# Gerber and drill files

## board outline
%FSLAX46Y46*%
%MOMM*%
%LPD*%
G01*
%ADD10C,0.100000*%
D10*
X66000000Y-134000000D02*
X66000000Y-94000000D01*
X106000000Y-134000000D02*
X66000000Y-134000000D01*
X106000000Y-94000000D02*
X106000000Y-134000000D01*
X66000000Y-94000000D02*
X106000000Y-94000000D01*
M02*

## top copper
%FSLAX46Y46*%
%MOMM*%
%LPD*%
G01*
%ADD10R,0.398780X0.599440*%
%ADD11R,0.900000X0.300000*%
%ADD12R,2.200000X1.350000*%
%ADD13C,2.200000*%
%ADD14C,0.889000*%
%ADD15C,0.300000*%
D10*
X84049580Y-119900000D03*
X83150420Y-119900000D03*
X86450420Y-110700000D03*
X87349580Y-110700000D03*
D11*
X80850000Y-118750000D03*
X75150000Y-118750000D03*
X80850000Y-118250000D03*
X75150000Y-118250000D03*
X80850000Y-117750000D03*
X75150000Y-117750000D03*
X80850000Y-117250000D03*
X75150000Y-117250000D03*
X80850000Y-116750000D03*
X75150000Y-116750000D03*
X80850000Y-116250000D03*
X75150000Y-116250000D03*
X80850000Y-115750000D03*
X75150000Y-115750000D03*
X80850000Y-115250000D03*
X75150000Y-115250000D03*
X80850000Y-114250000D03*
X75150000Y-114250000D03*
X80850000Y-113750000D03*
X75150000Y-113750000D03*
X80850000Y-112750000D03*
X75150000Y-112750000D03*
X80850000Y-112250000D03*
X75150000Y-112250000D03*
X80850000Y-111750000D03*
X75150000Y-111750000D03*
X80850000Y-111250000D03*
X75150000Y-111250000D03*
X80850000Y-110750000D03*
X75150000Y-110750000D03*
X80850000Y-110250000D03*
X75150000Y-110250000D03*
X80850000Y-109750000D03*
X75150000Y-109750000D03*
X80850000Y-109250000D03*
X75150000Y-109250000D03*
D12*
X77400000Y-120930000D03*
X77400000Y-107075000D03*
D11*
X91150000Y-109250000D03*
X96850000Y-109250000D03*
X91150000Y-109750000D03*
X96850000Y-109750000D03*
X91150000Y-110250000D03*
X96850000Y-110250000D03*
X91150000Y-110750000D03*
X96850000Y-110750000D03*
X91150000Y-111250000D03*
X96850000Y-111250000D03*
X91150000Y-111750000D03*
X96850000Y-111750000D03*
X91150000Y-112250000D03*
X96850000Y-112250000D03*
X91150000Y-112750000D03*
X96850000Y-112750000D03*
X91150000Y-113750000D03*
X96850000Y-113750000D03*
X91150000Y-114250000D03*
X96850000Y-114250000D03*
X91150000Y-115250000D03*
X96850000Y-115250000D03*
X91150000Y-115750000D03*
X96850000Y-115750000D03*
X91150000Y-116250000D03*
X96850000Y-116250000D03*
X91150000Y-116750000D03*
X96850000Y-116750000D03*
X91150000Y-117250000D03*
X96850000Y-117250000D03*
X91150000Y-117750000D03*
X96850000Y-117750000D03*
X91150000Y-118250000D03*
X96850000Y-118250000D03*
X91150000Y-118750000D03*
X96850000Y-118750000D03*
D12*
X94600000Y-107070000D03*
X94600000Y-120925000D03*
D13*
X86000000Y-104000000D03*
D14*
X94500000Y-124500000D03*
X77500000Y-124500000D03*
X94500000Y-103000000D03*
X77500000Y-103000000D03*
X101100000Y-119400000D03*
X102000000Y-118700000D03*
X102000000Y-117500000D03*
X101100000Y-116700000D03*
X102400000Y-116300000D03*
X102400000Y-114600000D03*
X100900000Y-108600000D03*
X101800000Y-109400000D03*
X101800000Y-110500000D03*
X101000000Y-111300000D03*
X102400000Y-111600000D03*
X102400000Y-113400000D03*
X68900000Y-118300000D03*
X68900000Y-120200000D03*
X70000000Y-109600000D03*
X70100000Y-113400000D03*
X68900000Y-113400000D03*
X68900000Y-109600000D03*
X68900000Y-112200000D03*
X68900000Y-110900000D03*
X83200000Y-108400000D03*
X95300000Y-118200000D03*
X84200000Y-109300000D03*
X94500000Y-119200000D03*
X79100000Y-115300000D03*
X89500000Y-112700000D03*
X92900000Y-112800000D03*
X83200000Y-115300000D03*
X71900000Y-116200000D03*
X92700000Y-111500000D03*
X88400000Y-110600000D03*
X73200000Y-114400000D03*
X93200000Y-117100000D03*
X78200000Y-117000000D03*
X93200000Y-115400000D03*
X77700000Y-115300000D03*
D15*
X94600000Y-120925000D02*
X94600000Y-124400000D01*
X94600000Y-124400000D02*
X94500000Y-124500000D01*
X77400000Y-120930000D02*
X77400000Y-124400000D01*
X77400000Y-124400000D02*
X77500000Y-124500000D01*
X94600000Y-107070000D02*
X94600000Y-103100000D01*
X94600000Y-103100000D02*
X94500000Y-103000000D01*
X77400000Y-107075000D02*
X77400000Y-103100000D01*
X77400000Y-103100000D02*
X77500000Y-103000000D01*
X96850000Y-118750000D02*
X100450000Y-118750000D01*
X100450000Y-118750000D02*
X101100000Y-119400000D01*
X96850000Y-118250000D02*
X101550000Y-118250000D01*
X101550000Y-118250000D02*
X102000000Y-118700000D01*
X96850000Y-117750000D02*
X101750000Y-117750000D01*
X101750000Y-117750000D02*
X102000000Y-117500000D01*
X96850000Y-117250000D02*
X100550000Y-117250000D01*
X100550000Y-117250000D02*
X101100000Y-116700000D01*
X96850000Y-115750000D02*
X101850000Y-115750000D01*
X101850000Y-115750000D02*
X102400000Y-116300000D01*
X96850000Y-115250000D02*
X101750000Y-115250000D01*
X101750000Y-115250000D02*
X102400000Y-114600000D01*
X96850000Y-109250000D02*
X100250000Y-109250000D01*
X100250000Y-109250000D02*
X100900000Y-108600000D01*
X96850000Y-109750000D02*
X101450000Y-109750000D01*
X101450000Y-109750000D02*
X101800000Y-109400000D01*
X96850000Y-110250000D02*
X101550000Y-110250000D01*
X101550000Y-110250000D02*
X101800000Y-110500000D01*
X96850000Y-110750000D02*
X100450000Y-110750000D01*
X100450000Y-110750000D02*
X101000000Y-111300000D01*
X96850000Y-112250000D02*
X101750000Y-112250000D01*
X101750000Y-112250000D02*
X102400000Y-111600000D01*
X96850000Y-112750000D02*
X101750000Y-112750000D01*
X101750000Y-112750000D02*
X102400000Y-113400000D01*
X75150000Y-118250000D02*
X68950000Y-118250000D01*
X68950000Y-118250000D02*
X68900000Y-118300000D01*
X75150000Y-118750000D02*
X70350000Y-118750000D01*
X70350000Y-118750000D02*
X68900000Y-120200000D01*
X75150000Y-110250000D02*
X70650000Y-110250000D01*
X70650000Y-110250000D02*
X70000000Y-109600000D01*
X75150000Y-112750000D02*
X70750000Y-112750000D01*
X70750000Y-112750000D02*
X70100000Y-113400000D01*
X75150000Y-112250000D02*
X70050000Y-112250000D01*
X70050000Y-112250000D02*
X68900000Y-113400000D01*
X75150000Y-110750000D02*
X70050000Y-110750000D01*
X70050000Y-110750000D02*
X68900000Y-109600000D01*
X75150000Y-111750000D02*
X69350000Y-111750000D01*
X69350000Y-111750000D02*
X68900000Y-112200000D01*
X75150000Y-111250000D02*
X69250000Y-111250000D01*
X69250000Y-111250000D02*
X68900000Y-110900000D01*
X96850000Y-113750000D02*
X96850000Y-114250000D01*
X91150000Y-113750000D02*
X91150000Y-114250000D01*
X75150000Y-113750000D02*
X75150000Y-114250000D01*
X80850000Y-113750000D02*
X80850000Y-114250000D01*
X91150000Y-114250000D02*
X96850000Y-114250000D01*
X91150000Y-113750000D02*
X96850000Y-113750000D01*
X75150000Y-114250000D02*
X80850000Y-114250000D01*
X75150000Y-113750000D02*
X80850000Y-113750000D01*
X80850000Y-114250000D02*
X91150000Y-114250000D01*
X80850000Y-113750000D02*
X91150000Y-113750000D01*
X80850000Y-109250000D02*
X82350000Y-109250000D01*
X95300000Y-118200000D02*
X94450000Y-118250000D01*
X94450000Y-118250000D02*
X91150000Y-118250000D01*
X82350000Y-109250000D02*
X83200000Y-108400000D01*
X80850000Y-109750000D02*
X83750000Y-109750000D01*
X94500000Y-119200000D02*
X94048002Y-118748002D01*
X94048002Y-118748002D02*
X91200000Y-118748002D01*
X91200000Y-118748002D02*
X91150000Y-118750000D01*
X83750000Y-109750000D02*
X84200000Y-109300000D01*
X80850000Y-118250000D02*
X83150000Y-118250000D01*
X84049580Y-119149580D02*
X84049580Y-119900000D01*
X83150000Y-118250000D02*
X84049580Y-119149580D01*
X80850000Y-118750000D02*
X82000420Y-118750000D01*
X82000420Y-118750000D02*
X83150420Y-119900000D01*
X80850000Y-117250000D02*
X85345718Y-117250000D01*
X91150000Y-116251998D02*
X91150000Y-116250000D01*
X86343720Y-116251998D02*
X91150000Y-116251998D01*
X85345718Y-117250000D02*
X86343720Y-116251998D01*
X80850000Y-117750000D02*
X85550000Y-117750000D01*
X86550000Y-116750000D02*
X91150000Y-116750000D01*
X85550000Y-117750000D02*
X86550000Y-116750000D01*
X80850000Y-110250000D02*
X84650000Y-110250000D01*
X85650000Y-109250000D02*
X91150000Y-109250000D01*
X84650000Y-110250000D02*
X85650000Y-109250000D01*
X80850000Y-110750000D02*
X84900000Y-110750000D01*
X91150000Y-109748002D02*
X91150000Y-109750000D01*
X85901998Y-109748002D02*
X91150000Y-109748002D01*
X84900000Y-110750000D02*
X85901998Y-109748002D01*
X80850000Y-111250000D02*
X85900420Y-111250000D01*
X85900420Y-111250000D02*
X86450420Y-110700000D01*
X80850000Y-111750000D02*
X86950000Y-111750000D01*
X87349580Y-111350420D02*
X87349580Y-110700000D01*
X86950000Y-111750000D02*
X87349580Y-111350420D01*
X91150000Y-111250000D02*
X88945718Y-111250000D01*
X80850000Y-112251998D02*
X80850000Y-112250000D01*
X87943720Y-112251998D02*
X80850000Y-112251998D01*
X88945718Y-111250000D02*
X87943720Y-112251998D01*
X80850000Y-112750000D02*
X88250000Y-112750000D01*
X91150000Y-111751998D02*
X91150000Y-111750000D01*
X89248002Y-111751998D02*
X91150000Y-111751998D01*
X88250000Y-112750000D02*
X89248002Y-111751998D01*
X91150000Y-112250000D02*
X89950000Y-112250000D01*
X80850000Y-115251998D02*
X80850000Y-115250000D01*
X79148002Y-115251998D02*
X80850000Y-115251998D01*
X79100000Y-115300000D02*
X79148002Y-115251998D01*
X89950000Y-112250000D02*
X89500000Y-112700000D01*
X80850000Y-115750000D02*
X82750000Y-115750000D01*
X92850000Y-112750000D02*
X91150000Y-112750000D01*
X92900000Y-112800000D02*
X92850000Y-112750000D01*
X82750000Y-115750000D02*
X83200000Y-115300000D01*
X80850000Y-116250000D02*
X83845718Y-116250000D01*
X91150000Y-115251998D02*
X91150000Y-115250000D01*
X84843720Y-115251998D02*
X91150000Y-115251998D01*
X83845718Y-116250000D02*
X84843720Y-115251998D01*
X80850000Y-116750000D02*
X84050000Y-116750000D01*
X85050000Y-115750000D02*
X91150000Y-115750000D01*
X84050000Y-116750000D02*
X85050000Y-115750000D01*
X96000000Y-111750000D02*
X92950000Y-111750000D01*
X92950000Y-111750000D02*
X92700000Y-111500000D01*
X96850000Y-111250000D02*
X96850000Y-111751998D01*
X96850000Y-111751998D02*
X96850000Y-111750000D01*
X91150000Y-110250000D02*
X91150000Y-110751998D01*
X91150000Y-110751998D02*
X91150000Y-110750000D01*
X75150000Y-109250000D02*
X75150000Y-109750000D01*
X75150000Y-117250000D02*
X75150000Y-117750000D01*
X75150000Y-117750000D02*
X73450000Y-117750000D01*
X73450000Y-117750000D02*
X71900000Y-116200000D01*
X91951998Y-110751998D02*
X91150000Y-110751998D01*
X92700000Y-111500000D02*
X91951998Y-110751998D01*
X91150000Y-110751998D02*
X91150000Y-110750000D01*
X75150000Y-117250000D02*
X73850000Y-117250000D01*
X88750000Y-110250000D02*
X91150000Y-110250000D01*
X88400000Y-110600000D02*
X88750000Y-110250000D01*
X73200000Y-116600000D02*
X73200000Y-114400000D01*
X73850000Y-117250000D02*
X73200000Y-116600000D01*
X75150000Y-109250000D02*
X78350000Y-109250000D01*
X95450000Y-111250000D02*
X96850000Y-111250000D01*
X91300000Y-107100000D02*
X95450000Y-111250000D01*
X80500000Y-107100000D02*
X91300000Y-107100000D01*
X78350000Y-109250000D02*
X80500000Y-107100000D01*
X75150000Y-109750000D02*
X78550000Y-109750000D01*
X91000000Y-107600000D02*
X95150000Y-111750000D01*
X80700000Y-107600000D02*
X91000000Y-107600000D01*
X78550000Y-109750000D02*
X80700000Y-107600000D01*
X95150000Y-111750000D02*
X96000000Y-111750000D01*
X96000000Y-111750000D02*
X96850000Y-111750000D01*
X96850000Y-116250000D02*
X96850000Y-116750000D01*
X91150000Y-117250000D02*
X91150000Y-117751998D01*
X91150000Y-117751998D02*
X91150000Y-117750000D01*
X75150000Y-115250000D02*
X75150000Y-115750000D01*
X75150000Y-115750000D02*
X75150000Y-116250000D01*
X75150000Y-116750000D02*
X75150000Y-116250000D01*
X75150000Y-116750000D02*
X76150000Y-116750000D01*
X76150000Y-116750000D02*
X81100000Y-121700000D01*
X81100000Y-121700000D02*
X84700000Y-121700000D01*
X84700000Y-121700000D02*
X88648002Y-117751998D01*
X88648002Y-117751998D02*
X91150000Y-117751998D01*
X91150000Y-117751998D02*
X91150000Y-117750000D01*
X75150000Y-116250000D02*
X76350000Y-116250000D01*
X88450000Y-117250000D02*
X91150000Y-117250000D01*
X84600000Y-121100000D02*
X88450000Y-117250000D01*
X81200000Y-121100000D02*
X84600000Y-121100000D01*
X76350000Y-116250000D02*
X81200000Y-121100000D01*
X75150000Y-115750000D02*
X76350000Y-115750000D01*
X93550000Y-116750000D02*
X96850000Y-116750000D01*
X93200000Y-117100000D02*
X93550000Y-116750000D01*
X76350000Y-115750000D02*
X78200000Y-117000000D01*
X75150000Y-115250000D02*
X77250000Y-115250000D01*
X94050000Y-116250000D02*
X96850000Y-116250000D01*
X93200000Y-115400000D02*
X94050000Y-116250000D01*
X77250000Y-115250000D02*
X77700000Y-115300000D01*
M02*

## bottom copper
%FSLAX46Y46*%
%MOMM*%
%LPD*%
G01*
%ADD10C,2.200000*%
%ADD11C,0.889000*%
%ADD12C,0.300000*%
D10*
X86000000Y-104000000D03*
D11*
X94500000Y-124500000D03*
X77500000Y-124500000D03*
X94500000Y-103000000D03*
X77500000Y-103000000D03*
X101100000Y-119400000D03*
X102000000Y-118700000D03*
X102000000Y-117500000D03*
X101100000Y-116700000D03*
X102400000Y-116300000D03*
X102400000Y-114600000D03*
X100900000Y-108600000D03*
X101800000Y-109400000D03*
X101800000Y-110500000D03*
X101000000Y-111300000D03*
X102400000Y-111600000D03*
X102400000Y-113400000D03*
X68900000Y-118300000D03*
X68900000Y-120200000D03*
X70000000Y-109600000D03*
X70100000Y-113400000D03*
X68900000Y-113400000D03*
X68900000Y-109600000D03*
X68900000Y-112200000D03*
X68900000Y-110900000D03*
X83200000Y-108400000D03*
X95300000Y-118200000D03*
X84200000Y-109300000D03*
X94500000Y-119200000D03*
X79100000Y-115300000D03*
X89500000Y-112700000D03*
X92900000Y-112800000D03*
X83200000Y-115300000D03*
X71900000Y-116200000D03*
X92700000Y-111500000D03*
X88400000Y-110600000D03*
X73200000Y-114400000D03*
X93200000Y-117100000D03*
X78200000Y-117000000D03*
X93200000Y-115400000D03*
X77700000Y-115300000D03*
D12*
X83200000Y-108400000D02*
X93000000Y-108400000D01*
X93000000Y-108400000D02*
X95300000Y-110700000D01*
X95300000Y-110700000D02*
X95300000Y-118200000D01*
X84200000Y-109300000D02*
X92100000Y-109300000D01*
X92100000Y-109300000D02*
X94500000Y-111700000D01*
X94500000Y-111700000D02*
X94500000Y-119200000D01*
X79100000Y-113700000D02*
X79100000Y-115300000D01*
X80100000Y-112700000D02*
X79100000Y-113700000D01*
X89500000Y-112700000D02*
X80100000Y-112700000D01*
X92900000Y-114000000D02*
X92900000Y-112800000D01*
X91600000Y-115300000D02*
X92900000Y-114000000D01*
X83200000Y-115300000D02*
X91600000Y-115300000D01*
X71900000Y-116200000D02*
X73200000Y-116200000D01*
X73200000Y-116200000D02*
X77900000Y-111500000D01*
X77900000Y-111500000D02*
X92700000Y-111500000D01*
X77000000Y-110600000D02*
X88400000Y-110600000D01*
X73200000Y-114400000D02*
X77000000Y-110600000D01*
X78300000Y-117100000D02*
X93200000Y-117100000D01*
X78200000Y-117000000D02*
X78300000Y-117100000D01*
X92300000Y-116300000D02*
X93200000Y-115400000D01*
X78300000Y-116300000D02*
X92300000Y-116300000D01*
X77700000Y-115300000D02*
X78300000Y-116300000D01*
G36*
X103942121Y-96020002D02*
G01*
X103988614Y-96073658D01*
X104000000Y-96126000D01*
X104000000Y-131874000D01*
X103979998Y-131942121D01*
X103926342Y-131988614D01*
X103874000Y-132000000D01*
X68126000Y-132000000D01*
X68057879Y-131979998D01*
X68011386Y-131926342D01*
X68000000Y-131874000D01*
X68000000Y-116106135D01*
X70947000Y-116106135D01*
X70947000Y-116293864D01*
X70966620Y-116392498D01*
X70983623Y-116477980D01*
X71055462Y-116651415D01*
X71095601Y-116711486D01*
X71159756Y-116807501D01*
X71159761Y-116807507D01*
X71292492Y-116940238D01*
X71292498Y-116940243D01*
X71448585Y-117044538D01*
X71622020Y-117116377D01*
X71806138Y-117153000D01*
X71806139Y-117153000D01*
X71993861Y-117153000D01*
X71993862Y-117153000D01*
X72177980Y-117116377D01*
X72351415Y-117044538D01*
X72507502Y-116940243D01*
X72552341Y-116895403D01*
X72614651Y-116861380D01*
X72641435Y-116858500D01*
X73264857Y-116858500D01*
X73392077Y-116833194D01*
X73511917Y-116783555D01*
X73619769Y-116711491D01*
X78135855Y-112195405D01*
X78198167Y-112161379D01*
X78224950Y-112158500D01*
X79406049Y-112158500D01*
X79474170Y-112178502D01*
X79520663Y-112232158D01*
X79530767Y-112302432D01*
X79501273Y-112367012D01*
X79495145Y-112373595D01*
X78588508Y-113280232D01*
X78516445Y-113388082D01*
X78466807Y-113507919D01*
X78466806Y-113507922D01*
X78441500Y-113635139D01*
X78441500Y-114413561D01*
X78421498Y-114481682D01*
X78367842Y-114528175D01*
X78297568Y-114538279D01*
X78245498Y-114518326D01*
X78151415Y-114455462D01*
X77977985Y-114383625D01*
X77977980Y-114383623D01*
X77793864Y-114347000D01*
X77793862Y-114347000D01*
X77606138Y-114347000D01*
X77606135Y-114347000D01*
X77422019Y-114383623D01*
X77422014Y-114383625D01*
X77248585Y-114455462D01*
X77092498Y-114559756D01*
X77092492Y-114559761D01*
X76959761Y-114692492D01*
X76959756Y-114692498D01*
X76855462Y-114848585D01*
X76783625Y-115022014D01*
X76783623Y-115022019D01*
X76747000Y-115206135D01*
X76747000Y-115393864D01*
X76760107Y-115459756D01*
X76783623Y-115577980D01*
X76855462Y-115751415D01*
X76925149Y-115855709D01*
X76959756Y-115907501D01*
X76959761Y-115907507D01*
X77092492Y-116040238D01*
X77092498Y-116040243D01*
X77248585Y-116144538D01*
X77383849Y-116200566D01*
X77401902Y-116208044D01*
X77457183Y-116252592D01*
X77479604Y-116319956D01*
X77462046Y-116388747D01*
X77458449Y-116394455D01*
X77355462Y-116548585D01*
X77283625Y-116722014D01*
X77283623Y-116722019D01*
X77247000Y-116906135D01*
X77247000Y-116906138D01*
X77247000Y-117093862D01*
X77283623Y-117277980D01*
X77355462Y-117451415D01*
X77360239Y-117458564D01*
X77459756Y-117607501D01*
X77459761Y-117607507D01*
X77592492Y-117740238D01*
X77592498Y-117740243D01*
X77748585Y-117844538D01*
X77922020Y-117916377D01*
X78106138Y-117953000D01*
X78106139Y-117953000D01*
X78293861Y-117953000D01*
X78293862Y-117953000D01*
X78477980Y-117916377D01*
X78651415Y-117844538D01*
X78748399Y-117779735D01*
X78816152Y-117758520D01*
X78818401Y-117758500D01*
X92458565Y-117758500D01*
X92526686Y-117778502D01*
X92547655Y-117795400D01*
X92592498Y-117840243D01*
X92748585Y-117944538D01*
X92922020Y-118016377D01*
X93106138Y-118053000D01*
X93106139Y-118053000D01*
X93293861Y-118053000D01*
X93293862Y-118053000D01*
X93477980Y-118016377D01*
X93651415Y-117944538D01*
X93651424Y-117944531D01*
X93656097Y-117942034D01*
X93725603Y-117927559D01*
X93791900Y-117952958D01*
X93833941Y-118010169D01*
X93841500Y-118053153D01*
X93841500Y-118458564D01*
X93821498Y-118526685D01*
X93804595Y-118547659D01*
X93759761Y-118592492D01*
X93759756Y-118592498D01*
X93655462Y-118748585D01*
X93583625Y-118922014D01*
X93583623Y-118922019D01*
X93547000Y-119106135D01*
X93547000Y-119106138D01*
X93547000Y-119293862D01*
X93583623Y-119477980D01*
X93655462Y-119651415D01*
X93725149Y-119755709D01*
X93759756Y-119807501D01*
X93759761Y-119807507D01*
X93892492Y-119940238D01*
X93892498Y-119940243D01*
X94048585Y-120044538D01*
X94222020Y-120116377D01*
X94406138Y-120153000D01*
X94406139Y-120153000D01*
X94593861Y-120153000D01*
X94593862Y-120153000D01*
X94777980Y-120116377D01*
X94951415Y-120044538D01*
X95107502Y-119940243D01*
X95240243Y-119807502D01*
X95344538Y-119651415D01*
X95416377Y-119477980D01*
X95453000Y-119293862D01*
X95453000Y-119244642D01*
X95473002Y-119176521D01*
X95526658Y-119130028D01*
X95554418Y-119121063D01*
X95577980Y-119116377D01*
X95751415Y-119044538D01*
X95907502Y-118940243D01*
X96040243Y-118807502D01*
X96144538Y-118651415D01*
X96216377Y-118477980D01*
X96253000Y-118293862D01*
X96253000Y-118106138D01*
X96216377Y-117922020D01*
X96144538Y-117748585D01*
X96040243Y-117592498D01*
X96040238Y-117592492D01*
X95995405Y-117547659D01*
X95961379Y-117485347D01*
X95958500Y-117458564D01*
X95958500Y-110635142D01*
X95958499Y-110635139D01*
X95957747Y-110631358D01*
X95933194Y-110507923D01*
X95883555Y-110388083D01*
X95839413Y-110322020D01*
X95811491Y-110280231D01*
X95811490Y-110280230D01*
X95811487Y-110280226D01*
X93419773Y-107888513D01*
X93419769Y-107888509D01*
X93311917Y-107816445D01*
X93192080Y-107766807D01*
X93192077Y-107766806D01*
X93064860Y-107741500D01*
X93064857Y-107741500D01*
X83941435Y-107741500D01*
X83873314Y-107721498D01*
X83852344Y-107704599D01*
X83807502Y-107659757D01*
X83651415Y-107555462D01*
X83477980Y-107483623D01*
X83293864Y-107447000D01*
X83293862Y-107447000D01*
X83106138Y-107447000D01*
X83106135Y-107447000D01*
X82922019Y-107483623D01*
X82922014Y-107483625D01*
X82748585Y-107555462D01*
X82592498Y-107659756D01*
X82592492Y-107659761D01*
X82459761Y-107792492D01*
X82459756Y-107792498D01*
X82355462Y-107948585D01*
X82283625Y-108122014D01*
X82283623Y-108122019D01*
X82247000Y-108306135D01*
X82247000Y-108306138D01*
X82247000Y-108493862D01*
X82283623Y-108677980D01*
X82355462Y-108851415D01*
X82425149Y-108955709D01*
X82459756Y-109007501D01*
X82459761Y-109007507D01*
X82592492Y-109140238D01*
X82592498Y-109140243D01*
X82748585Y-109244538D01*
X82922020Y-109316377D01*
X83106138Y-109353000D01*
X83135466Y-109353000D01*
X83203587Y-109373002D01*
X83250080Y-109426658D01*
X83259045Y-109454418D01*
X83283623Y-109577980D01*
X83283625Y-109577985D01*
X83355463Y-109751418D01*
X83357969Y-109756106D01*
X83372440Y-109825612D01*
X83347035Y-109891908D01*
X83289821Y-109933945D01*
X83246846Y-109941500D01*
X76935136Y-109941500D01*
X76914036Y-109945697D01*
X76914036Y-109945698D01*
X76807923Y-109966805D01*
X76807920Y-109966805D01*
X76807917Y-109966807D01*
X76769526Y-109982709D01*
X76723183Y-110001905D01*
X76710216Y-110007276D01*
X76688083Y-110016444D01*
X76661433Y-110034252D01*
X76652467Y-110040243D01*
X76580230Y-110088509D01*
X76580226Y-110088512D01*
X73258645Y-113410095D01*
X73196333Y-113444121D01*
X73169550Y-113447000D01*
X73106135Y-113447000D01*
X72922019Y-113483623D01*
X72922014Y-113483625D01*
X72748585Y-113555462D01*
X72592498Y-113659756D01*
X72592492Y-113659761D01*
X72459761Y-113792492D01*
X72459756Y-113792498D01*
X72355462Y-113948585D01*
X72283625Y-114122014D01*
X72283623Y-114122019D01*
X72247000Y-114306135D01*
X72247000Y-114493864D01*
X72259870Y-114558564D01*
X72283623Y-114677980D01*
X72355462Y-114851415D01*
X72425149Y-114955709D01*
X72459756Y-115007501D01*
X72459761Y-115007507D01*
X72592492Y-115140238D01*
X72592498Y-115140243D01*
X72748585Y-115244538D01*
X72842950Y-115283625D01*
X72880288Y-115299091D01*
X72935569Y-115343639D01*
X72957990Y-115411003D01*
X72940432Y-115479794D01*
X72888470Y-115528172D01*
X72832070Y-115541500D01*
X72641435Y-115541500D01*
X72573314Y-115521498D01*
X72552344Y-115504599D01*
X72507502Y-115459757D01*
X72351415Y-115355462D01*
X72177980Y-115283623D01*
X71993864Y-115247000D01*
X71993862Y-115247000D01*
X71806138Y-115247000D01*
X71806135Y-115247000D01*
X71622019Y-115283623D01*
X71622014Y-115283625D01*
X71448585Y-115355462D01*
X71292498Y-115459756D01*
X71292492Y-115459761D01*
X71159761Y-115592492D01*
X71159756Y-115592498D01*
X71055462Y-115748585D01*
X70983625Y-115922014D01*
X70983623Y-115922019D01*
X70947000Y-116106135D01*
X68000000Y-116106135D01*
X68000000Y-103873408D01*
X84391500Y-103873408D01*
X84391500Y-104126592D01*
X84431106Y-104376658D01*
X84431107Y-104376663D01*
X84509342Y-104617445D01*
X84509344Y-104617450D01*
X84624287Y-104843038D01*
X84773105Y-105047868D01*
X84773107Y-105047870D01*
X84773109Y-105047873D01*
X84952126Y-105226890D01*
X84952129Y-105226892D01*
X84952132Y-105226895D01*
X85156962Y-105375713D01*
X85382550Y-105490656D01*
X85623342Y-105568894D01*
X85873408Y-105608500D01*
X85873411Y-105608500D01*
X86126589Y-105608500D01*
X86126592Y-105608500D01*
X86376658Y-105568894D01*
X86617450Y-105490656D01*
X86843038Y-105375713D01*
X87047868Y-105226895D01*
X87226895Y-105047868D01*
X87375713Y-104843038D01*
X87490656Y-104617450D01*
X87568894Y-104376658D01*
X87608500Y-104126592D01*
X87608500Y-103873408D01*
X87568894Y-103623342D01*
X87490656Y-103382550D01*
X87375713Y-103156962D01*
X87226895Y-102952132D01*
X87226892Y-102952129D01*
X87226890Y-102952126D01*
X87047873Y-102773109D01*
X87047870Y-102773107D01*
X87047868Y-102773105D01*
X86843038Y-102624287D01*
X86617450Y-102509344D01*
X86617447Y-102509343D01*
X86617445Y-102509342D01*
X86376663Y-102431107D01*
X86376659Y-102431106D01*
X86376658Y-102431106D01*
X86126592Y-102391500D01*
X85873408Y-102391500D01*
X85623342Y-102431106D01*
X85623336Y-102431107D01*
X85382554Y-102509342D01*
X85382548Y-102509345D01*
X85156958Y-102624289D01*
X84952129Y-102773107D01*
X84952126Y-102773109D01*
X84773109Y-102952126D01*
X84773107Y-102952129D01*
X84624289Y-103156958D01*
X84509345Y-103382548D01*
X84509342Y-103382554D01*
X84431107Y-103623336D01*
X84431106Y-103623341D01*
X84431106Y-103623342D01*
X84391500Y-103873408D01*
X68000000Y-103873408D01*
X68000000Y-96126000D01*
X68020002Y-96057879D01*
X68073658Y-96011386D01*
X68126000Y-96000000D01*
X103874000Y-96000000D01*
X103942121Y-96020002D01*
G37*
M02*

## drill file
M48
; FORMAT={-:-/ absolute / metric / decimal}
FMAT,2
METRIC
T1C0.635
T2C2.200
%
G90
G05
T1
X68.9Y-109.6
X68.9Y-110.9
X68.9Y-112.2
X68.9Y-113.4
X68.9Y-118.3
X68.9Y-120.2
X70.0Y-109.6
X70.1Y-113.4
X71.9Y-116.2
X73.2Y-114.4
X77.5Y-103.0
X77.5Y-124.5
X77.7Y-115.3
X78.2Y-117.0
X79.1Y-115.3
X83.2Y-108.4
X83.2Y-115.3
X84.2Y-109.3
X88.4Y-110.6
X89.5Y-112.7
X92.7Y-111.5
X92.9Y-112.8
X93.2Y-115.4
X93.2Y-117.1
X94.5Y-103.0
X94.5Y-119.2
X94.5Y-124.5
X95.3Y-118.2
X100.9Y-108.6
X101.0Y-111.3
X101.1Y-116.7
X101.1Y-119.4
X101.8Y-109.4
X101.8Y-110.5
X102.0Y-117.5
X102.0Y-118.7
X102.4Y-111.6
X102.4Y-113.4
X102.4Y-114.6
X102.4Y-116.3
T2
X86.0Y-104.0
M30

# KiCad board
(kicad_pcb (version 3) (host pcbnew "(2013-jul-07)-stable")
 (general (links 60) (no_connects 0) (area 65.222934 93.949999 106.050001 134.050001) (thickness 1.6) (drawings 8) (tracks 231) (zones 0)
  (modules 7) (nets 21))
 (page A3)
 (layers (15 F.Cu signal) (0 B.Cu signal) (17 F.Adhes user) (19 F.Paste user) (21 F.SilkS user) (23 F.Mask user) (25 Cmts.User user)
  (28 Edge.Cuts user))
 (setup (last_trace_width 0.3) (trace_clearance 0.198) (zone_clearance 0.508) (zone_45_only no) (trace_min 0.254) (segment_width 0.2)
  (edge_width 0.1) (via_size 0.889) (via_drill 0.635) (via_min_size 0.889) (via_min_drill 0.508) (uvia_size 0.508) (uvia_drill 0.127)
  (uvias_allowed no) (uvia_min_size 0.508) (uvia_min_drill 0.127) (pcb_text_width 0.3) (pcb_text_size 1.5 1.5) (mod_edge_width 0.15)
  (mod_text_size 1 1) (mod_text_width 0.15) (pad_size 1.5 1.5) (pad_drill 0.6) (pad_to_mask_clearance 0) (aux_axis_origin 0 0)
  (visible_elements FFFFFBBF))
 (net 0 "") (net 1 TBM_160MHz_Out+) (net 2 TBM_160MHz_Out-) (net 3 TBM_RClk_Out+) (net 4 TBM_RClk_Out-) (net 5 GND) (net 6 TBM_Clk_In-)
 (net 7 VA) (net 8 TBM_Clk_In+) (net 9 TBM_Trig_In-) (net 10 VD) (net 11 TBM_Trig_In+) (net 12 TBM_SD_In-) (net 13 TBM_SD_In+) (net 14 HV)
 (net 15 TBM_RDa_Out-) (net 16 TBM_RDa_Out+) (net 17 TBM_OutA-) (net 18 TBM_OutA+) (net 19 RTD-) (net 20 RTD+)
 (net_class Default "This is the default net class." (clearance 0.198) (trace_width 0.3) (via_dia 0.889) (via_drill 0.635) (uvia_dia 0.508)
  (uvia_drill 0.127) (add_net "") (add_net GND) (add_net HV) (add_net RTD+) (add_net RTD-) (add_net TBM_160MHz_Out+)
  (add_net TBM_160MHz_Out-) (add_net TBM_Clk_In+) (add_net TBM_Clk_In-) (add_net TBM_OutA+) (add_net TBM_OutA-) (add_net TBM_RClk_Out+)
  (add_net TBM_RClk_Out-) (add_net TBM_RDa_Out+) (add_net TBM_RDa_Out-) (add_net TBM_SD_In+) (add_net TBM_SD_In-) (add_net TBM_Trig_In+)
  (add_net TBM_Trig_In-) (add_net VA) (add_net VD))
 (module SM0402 (layer F.Cu) (at 83.6 119.9 180)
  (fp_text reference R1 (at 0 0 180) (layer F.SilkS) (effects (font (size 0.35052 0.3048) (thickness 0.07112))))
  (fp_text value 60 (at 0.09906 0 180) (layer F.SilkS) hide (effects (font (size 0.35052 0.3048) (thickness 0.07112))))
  (pad 1 smd rect (at -0.44958 0 180) (size 0.39878 0.59944) (layers F.Cu F.Paste F.Mask) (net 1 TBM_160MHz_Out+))
  (pad 2 smd rect (at 0.44958 0 180) (size 0.39878 0.59944) (layers F.Cu F.Paste F.Mask) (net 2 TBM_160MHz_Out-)))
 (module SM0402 (layer F.Cu) (at 86.9 110.7)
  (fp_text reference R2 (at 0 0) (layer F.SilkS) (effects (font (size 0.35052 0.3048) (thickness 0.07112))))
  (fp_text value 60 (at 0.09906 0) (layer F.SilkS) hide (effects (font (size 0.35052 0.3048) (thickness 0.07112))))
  (pad 1 smd rect (at -0.44958 0) (size 0.39878 0.59944) (layers F.Cu F.Paste F.Mask) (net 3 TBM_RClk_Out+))
  (pad 2 smd rect (at 0.44958 0) (size 0.39878 0.59944) (layers F.Cu F.Paste F.Mask) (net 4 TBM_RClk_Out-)))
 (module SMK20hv (layer F.Cu) (at 78 114 90)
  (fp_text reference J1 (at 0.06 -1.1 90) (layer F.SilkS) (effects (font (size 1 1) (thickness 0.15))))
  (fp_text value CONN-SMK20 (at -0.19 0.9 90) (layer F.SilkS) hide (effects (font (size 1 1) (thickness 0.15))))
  (pad 1 smd rect (at -4.75 2.85 90) (size 0.3 0.9) (layers F.Cu F.Paste F.Mask) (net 2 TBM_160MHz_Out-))
  (pad 2 smd rect (at -4.75 -2.85 90) (size 0.3 0.9) (layers F.Cu F.Paste F.Mask) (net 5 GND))
  (pad 3 smd rect (at -4.25 2.85 90) (size 0.3 0.9) (layers F.Cu F.Paste F.Mask) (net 1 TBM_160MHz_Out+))
  (pad 4 smd rect (at -4.25 -2.85 90) (size 0.3 0.9) (layers F.Cu F.Paste F.Mask) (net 5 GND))
  (pad 5 smd rect (at -3.75 2.85 90) (size 0.3 0.9) (layers F.Cu F.Paste F.Mask) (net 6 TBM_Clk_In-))
  (pad 6 smd rect (at -3.75 -2.85 90) (size 0.3 0.9) (layers F.Cu F.Paste F.Mask) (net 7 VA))
  (pad 7 smd rect (at -3.25 2.85 90) (size 0.3 0.9) (layers F.Cu F.Paste F.Mask) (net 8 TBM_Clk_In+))
  (pad 8 smd rect (at -3.25 -2.85 90) (size 0.3 0.9) (layers F.Cu F.Paste F.Mask) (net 7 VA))
  (pad 9 smd rect (at -2.75 2.85 90) (size 0.3 0.9) (layers F.Cu F.Paste F.Mask) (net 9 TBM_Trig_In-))
  (pad 10 smd rect (at -2.75 -2.85 90) (size 0.3 0.9) (layers F.Cu F.Paste F.Mask) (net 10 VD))
  (pad 11 smd rect (at -2.25 2.85 90) (size 0.3 0.9) (layers F.Cu F.Paste F.Mask) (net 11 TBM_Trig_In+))
  (pad 12 smd rect (at -2.25 -2.85 90) (size 0.3 0.9) (layers F.Cu F.Paste F.Mask) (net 10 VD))
  (pad 13 smd rect (at -1.75 2.85 90) (size 0.3 0.9) (layers F.Cu F.Paste F.Mask) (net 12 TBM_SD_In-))
  (pad 14 smd rect (at -1.75 -2.85 90) (size 0.3 0.9) (layers F.Cu F.Paste F.Mask) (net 10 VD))
  (pad 15 smd rect (at -1.25 2.85 90) (size 0.3 0.9) (layers F.Cu F.Paste F.Mask) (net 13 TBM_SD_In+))
  (pad 16 smd rect (at -1.25 -2.85 90) (size 0.3 0.9) (layers F.Cu F.Paste F.Mask) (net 10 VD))
  (pad 19 smd rect (at -0.25 2.85 90) (size 0.3 0.9) (layers F.Cu F.Paste F.Mask) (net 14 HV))
  (pad 20 smd rect (at -0.25 -2.85 90) (size 0.3 0.9) (layers F.Cu F.Paste F.Mask) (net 14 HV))
  (pad 21 smd rect (at 0.25 2.85 90) (size 0.3 0.9) (layers F.Cu F.Paste F.Mask) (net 14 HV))
  (pad 22 smd rect (at 0.25 -2.85 90) (size 0.3 0.9) (layers F.Cu F.Paste F.Mask) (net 14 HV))
  (pad 25 smd rect (at 1.25 2.85 90) (size 0.3 0.9) (layers F.Cu F.Paste F.Mask) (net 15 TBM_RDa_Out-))
  (pad 26 smd rect (at 1.25 -2.85 90) (size 0.3 0.9) (layers F.Cu F.Paste F.Mask) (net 5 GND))
  (pad 27 smd rect (at 1.75 2.85 90) (size 0.3 0.9) (layers F.Cu F.Paste F.Mask) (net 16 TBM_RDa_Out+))
  (pad 28 smd rect (at 1.75 -2.85 90) (size 0.3 0.9) (layers F.Cu F.Paste F.Mask) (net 5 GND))
  (pad 29 smd rect (at 2.25 2.85 90) (size 0.3 0.9) (layers F.Cu F.Paste F.Mask) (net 4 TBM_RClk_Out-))
  (pad 30 smd rect (at 2.25 -2.85 90) (size 0.3 0.9) (layers F.Cu F.Paste F.Mask) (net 5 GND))
  (pad 31 smd rect (at 2.75 2.85 90) (size 0.3 0.9) (layers F.Cu F.Paste F.Mask) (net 3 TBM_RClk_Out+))
  (pad 32 smd rect (at 2.75 -2.85 90) (size 0.3 0.9) (layers F.Cu F.Paste F.Mask) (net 5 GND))
  (pad 33 smd rect (at 3.25 2.85 90) (size 0.3 0.9) (layers F.Cu F.Paste F.Mask) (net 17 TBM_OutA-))
  (pad 34 smd rect (at 3.25 -2.85 90) (size 0.3 0.9) (layers F.Cu F.Paste F.Mask) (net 5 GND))
  (pad 35 smd rect (at 3.75 2.85 90) (size 0.3 0.9) (layers F.Cu F.Paste F.Mask) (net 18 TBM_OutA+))
  (pad 36 smd rect (at 3.75 -2.85 90) (size 0.3 0.9) (layers F.Cu F.Paste F.Mask) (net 5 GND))
  (pad 37 smd rect (at 4.25 2.85 90) (size 0.3 0.9) (layers F.Cu F.Paste F.Mask) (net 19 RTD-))
  (pad 38 smd rect (at 4.25 -2.85 90) (size 0.3 0.9) (layers F.Cu F.Paste F.Mask) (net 7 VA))
  (pad 39 smd rect (at 4.75 2.85 90) (size 0.3 0.9) (layers F.Cu F.Paste F.Mask) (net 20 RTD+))
  (pad 40 smd rect (at 4.75 -2.85 90) (size 0.3 0.9) (layers F.Cu F.Paste F.Mask) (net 7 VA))
  (pad 41 smd rect (at -6.93 -0.6 90) (size 1.35 2.2) (layers F.Cu F.Paste F.Mask) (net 5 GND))
  (pad 42 smd rect (at 6.925 -0.6 90) (size 1.35 2.2) (layers F.Cu F.Paste F.Mask) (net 5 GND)))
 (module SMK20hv (layer F.Cu) (at 94 114 270)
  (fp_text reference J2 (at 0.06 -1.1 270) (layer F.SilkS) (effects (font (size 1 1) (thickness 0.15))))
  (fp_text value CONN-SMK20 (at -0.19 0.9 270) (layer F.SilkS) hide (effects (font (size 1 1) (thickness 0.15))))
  (pad 1 smd rect (at -4.75 2.85 270) (size 0.3 0.9) (layers F.Cu F.Paste F.Mask) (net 18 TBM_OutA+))
  (pad 2 smd rect (at -4.75 -2.85 270) (size 0.3 0.9) (layers F.Cu F.Paste F.Mask) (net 5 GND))
  (pad 3 smd rect (at -4.25 2.85 270) (size 0.3 0.9) (layers F.Cu F.Paste F.Mask) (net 17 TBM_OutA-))
  (pad 4 smd rect (at -4.25 -2.85 270) (size 0.3 0.9) (layers F.Cu F.Paste F.Mask) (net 5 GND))
  (pad 5 smd rect (at -3.75 2.85 270) (size 0.3 0.9) (layers F.Cu F.Paste F.Mask) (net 7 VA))
  (pad 6 smd rect (at -3.75 -2.85 270) (size 0.3 0.9) (layers F.Cu F.Paste F.Mask) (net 5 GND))
  (pad 7 smd rect (at -3.25 2.85 270) (size 0.3 0.9) (layers F.Cu F.Paste F.Mask) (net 7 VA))
  (pad 8 smd rect (at -3.25 -2.85 270) (size 0.3 0.9) (layers F.Cu F.Paste F.Mask) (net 5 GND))
  (pad 9 smd rect (at -2.75 2.85 270) (size 0.3 0.9) (layers F.Cu F.Paste F.Mask) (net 16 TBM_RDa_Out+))
  (pad 10 smd rect (at -2.75 -2.85 270) (size 0.3 0.9) (layers F.Cu F.Paste F.Mask) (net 7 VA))
  (pad 11 smd rect (at -2.25 2.85 270) (size 0.3 0.9) (layers F.Cu F.Paste F.Mask) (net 15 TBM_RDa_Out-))
  (pad 12 smd rect (at -2.25 -2.85 270) (size 0.3 0.9) (layers F.Cu F.Paste F.Mask) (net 7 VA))
  (pad 13 smd rect (at -1.75 2.85 270) (size 0.3 0.9) (layers F.Cu F.Paste F.Mask) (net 13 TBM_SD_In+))
  (pad 14 smd rect (at -1.75 -2.85 270) (size 0.3 0.9) (layers F.Cu F.Paste F.Mask) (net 5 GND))
  (pad 15 smd rect (at -1.25 2.85 270) (size 0.3 0.9) (layers F.Cu F.Paste F.Mask) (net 12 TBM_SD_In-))
  (pad 16 smd rect (at -1.25 -2.85 270) (size 0.3 0.9) (layers F.Cu F.Paste F.Mask) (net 5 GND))
  (pad 19 smd rect (at -0.25 2.85 270) (size 0.3 0.9) (layers F.Cu F.Paste F.Mask) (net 14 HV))
  (pad 20 smd rect (at -0.25 -2.85 270) (size 0.3 0.9) (layers F.Cu F.Paste F.Mask) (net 14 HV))
  (pad 21 smd rect (at 0.25 2.85 270) (size 0.3 0.9) (layers F.Cu F.Paste F.Mask) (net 14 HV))
  (pad 22 smd rect (at 0.25 -2.85 270) (size 0.3 0.9) (layers F.Cu F.Paste F.Mask) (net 14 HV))
  (pad 25 smd rect (at 1.25 2.85 270) (size 0.3 0.9) (layers F.Cu F.Paste F.Mask) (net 11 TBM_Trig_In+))
  (pad 26 smd rect (at 1.25 -2.85 270) (size 0.3 0.9) (layers F.Cu F.Paste F.Mask) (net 5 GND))
  (pad 27 smd rect (at 1.75 2.85 270) (size 0.3 0.9) (layers F.Cu F.Paste F.Mask) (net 9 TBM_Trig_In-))
  (pad 28 smd rect (at 1.75 -2.85 270) (size 0.3 0.9) (layers F.Cu F.Paste F.Mask) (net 5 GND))
  (pad 29 smd rect (at 2.25 2.85 270) (size 0.3 0.9) (layers F.Cu F.Paste F.Mask) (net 8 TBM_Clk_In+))
  (pad 30 smd rect (at 2.25 -2.85 270) (size 0.3 0.9) (layers F.Cu F.Paste F.Mask) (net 10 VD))
  (pad 31 smd rect (at 2.75 2.85 270) (size 0.3 0.9) (layers F.Cu F.Paste F.Mask) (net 6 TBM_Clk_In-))
  (pad 32 smd rect (at 2.75 -2.85 270) (size 0.3 0.9) (layers F.Cu F.Paste F.Mask) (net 10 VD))
  (pad 33 smd rect (at 3.25 2.85 270) (size 0.3 0.9) (layers F.Cu F.Paste F.Mask) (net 10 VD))
  (pad 34 smd rect (at 3.25 -2.85 270) (size 0.3 0.9) (layers F.Cu F.Paste F.Mask) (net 5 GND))
  (pad 35 smd rect (at 3.75 2.85 270) (size 0.3 0.9) (layers F.Cu F.Paste F.Mask) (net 10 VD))
  (pad 36 smd rect (at 3.75 -2.85 270) (size 0.3 0.9) (layers F.Cu F.Paste F.Mask) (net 5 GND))
  (pad 37 smd rect (at 4.25 2.85 270) (size 0.3 0.9) (layers F.Cu F.Paste F.Mask) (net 20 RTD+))
  (pad 38 smd rect (at 4.25 -2.85 270) (size 0.3 0.9) (layers F.Cu F.Paste F.Mask) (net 5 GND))
  (pad 39 smd rect (at 4.75 2.85 270) (size 0.3 0.9) (layers F.Cu F.Paste F.Mask) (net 19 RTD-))
  (pad 40 smd rect (at 4.75 -2.85 270) (size 0.3 0.9) (layers F.Cu F.Paste F.Mask) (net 5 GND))
  (pad 41 smd rect (at -6.93 -0.6 270) (size 1.35 2.2) (layers F.Cu F.Paste F.Mask) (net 5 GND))
  (pad 42 smd rect (at 6.925 -0.6 270) (size 1.35 2.2) (layers F.Cu F.Paste F.Mask) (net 5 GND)))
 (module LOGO (layer F.Cu) (at 101 100)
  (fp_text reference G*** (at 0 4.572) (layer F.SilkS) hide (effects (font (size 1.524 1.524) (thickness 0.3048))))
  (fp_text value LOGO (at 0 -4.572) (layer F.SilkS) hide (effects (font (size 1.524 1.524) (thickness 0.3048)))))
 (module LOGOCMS (layer F.Cu) (at 71.5 100)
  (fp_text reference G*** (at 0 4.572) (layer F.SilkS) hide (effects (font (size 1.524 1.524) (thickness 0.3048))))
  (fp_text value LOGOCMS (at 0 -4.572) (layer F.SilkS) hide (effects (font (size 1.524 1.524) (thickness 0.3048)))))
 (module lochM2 (layer F.Cu) (at 86 104)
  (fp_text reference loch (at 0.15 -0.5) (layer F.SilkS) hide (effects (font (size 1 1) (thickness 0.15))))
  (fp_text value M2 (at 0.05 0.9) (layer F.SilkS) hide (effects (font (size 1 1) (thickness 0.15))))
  (pad 1 thru_hole circle (at 0 0) (size 2.2 2.2) (drill 2.2) (layers *.Cu *.Mask F.SilkS)))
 (gr_line (start 66 134) (end 66 94) (angle 90) (layer Edge.Cuts) (width 0.1))
 (gr_line (start 106 134) (end 66 134) (angle 90) (layer Edge.Cuts) (width 0.1))
 (gr_line (start 106 94) (end 106 134) (angle 90) (layer Edge.Cuts) (width 0.1))
 (gr_line (start 66 94) (end 106 94) (angle 90) (layer Edge.Cuts) (width 0.1))
 (segment (start 94.6 120.925) (end 94.6 124.4) (width 0.3) (layer F.Cu) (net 5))
 (via (at 94.5 124.5) (size 0.889) (layers F.Cu B.Cu) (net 5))
 (segment (start 94.6 124.4) (end 94.5 124.5) (width 0.3) (layer F.Cu) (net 5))
 (segment (start 77.4 120.93) (end 77.4 124.4) (width 0.3) (layer F.Cu) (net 5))
 (via (at 77.5 124.5) (size 0.889) (layers F.Cu B.Cu) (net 5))
 (segment (start 77.4 124.4) (end 77.5 124.5) (width 0.3) (layer F.Cu) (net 5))
 (segment (start 94.6 107.07) (end 94.6 103.1) (width 0.3) (layer F.Cu) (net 5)) (via (at 94.5 103) (size 0.889) (layers F.Cu B.Cu) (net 5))
 (segment (start 94.6 103.1) (end 94.5 103) (width 0.3) (layer F.Cu) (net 5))
 (segment (start 77.4 107.075) (end 77.4 103.1) (width 0.3) (layer F.Cu) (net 5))
 (via (at 77.5 103) (size 0.889) (layers F.Cu B.Cu) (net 5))
 (segment (start 77.4 103.1) (end 77.5 103) (width 0.3) (layer F.Cu) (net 5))
 (segment (start 96.85 118.75) (end 100.45 118.75) (width 0.3) (layer F.Cu) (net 5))
 (via (at 101.1 119.4) (size 0.889) (layers F.Cu B.Cu) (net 5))
 (segment (start 100.45 118.75) (end 101.1 119.4) (width 0.3) (layer F.Cu) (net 5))
 (segment (start 96.85 118.25) (end 101.55 118.25) (width 0.3) (layer F.Cu) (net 5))
 (via (at 102 118.7) (size 0.889) (layers F.Cu B.Cu) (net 5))
 (segment (start 101.55 118.25) (end 102 118.7) (width 0.3) (layer F.Cu) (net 5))
 (segment (start 96.85 117.75) (end 101.75 117.75) (width 0.3) (layer F.Cu) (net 5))
 (via (at 102 117.5) (size 0.889) (layers F.Cu B.Cu) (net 5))
 (segment (start 101.75 117.75) (end 102 117.5) (width 0.3) (layer F.Cu) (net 5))
 (segment (start 96.85 117.25) (end 100.55 117.25) (width 0.3) (layer F.Cu) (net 5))
 (via (at 101.1 116.7) (size 0.889) (layers F.Cu B.Cu) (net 5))
 (segment (start 100.55 117.25) (end 101.1 116.7) (width 0.3) (layer F.Cu) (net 5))
 (segment (start 96.85 115.75) (end 101.85 115.75) (width 0.3) (layer F.Cu) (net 5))
 (via (at 102.4 116.3) (size 0.889) (layers F.Cu B.Cu) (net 5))
 (segment (start 101.85 115.75) (end 102.4 116.3) (width 0.3) (layer F.Cu) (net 5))
 (segment (start 96.85 115.25) (end 101.75 115.25) (width 0.3) (layer F.Cu) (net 5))
 (via (at 102.4 114.6) (size 0.889) (layers F.Cu B.Cu) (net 5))
 (segment (start 101.75 115.25) (end 102.4 114.6) (width 0.3) (layer F.Cu) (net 5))
 (segment (start 96.85 109.25) (end 100.25 109.25) (width 0.3) (layer F.Cu) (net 5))
 (via (at 100.9 108.6) (size 0.889) (layers F.Cu B.Cu) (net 5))
 (segment (start 100.25 109.25) (end 100.9 108.6) (width 0.3) (layer F.Cu) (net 5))
 (segment (start 96.85 109.75) (end 101.45 109.75) (width 0.3) (layer F.Cu) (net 5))
 (via (at 101.8 109.4) (size 0.889) (layers F.Cu B.Cu) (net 5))
 (segment (start 101.45 109.75) (end 101.8 109.4) (width 0.3) (layer F.Cu) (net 5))
 (segment (start 96.85 110.25) (end 101.55 110.25) (width 0.3) (layer F.Cu) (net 5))
 (via (at 101.8 110.5) (size 0.889) (layers F.Cu B.Cu) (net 5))
 (segment (start 101.55 110.25) (end 101.8 110.5) (width 0.3) (layer F.Cu) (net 5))
 (segment (start 96.85 110.75) (end 100.45 110.75) (width 0.3) (layer F.Cu) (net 5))
 (via (at 101 111.3) (size 0.889) (layers F.Cu B.Cu) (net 5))
 (segment (start 100.45 110.75) (end 101 111.3) (width 0.3) (layer F.Cu) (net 5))
 (segment (start 96.85 112.25) (end 101.75 112.25) (width 0.3) (layer F.Cu) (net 5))
 (via (at 102.4 111.6) (size 0.889) (layers F.Cu B.Cu) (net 5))
 (segment (start 101.75 112.25) (end 102.4 111.6) (width 0.3) (layer F.Cu) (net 5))
 (segment (start 96.85 112.75) (end 101.75 112.75) (width 0.3) (layer F.Cu) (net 5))
 (via (at 102.4 113.4) (size 0.889) (layers F.Cu B.Cu) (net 5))
 (segment (start 101.75 112.75) (end 102.4 113.4) (width 0.3) (layer F.Cu) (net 5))
 (segment (start 75.15 118.25) (end 68.95 118.25) (width 0.3) (layer F.Cu) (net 5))
 (via (at 68.9 118.3) (size 0.889) (layers F.Cu B.Cu) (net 5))
 (segment (start 68.95 118.25) (end 68.9 118.3) (width 0.3) (layer F.Cu) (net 5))
 (segment (start 75.15 118.75) (end 70.35 118.75) (width 0.3) (layer F.Cu) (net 5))
 (via (at 68.9 120.2) (size 0.889) (layers F.Cu B.Cu) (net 5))
 (segment (start 70.35 118.75) (end 68.9 120.2) (width 0.3) (layer F.Cu) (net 5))
 (segment (start 75.15 110.25) (end 70.65 110.25) (width 0.3) (layer F.Cu) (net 5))
 (via (at 70 109.6) (size 0.889) (layers F.Cu B.Cu) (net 5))
 (segment (start 70.65 110.25) (end 70 109.6) (width 0.3) (layer F.Cu) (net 5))
 (segment (start 75.15 112.75) (end 70.75 112.75) (width 0.3) (layer F.Cu) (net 5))
 (via (at 70.1 113.4) (size 0.889) (layers F.Cu B.Cu) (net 5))
 (segment (start 70.75 112.75) (end 70.1 113.4) (width 0.3) (layer F.Cu) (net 5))
 (segment (start 75.15 112.25) (end 70.05 112.25) (width 0.3) (layer F.Cu) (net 5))
 (via (at 68.9 113.4) (size 0.889) (layers F.Cu B.Cu) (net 5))
 (segment (start 70.05 112.25) (end 68.9 113.4) (width 0.3) (layer F.Cu) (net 5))
 (segment (start 75.15 110.75) (end 70.05 110.75) (width 0.3) (layer F.Cu) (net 5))
 (via (at 68.9 109.6) (size 0.889) (layers F.Cu B.Cu) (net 5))
 (segment (start 70.05 110.75) (end 68.9 109.6) (width 0.3) (layer F.Cu) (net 5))
 (segment (start 75.15 111.75) (end 69.35 111.75) (width 0.3) (layer F.Cu) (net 5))
 (via (at 68.9 112.2) (size 0.889) (layers F.Cu B.Cu) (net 5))
 (segment (start 69.35 111.75) (end 68.9 112.2) (width 0.3) (layer F.Cu) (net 5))
 (segment (start 75.15 111.25) (end 69.25 111.25) (width 0.3) (layer F.Cu) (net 5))
 (via (at 68.9 110.9) (size 0.889) (layers F.Cu B.Cu) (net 5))
 (segment (start 69.25 111.25) (end 68.9 110.9) (width 0.3) (layer F.Cu) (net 5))
 (segment (start 96.85 113.75) (end 96.85 114.25) (width 0.3) (layer F.Cu) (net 14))
 (segment (start 91.15 113.75) (end 91.15 114.25) (width 0.3) (layer F.Cu) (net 14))
 (segment (start 75.15 113.75) (end 75.15 114.25) (width 0.3) (layer F.Cu) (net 14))
 (segment (start 80.85 113.75) (end 80.85 114.25) (width 0.3) (layer F.Cu) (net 14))
 (segment (start 91.15 114.25) (end 96.85 114.25) (width 0.3) (layer F.Cu) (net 14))
 (segment (start 91.15 113.75) (end 96.85 113.75) (width 0.3) (layer F.Cu) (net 14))
 (segment (start 75.15 114.25) (end 80.85 114.25) (width 0.3) (layer F.Cu) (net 14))
 (segment (start 75.15 113.75) (end 80.85 113.75) (width 0.3) (layer F.Cu) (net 14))
 (segment (start 80.85 114.25) (end 91.15 114.25) (width 0.3) (layer F.Cu) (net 14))
 (segment (start 80.85 113.75) (end 91.15 113.75) (width 0.3) (layer F.Cu) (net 14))
 (segment (start 80.85 109.25) (end 82.35 109.25) (width 0.3) (layer F.Cu) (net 20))
 (via (at 83.2 108.4) (size 0.889) (layers F.Cu B.Cu) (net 20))
 (segment (start 83.2 108.4) (end 93 108.4) (width 0.3) (layer B.Cu) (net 20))
 (segment (start 93 108.4) (end 95.3 110.7) (width 0.3) (layer B.Cu) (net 20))
 (segment (start 95.3 110.7) (end 95.3 118.2) (width 0.3) (layer B.Cu) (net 20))
 (via (at 95.3 118.2) (size 0.889) (layers F.Cu B.Cu) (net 20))
 (segment (start 95.3 118.2) (end 94.45 118.25) (width 0.3) (layer F.Cu) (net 20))
 (segment (start 94.45 118.25) (end 91.15 118.25) (width 0.3) (layer F.Cu) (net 20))
 (segment (start 82.35 109.25) (end 83.2 108.4) (width 0.3) (layer F.Cu) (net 20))
 (segment (start 80.85 109.75) (end 83.75 109.75) (width 0.3) (layer F.Cu) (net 19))
 (via (at 84.2 109.3) (size 0.889) (layers F.Cu B.Cu) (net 19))
 (segment (start 84.2 109.3) (end 92.1 109.3) (width 0.3) (layer B.Cu) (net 19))
 (segment (start 92.1 109.3) (end 94.5 111.7) (width 0.3) (layer B.Cu) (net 19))
 (segment (start 94.5 111.7) (end 94.5 119.2) (width 0.3) (layer B.Cu) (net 19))
 (via (at 94.5 119.2) (size 0.889) (layers F.Cu B.Cu) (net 19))
 (segment (start 94.5 119.2) (end 94.048002 118.748002) (width 0.3) (layer F.Cu) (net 19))
 (segment (start 94.048002 118.748002) (end 91.2 118.748002) (width 0.3) (layer F.Cu) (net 19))
 (segment (start 91.2 118.748002) (end 91.15 118.75) (width 0.3) (layer F.Cu) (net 19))
 (segment (start 83.75 109.75) (end 84.2 109.3) (width 0.3) (layer F.Cu) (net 19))
 (segment (start 80.85 118.25) (end 83.15 118.25) (width 0.3) (layer F.Cu) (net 1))
 (segment (start 84.04958 119.14958) (end 84.04958 119.9) (width 0.3) (layer F.Cu) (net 1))
 (segment (start 83.15 118.25) (end 84.04958 119.14958) (width 0.3) (layer F.Cu) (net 1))
 (segment (start 80.85 118.75) (end 82.00042 118.75) (width 0.3) (layer F.Cu) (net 2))
 (segment (start 82.00042 118.75) (end 83.15042 119.9) (width 0.3) (layer F.Cu) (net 2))
 (segment (start 80.85 117.25) (end 85.345718 117.25) (width 0.3) (layer F.Cu) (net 8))
 (segment (start 91.15 116.251998) (end 91.15 116.25) (width 0.3) (layer F.Cu) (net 8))
 (segment (start 86.34372 116.251998) (end 91.15 116.251998) (width 0.3) (layer F.Cu) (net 8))
 (segment (start 85.345718 117.25) (end 86.34372 116.251998) (width 0.3) (layer F.Cu) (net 8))
 (segment (start 80.85 117.75) (end 85.55 117.75) (width 0.3) (layer F.Cu) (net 6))
 (segment (start 86.55 116.75) (end 91.15 116.75) (width 0.3) (layer F.Cu) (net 6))
 (segment (start 85.55 117.75) (end 86.55 116.75) (width 0.3) (layer F.Cu) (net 6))
 (segment (start 80.85 110.25) (end 84.65 110.25) (width 0.3) (layer F.Cu) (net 18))
 (segment (start 85.65 109.25) (end 91.15 109.25) (width 0.3) (layer F.Cu) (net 18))
 (segment (start 84.65 110.25) (end 85.65 109.25) (width 0.3) (layer F.Cu) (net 18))
 (segment (start 80.85 110.75) (end 84.9 110.75) (width 0.3) (layer F.Cu) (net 17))
 (segment (start 91.15 109.748002) (end 91.15 109.75) (width 0.3) (layer F.Cu) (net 17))
 (segment (start 85.901998 109.748002) (end 91.15 109.748002) (width 0.3) (layer F.Cu) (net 17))
 (segment (start 84.9 110.75) (end 85.901998 109.748002) (width 0.3) (layer F.Cu) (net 17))
 (segment (start 80.85 111.25) (end 85.90042 111.25) (width 0.3) (layer F.Cu) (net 3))
 (segment (start 85.90042 111.25) (end 86.45042 110.7) (width 0.3) (layer F.Cu) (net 3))
 (segment (start 80.85 111.75) (end 86.95 111.75) (width 0.3) (layer F.Cu) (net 4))
 (segment (start 87.34958 111.35042) (end 87.34958 110.7) (width 0.3) (layer F.Cu) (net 4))
 (segment (start 86.95 111.75) (end 87.34958 111.35042) (width 0.3) (layer F.Cu) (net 4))
 (segment (start 91.15 111.25) (end 88.945718 111.25) (width 0.3) (layer F.Cu) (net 16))
 (segment (start 80.85 112.251998) (end 80.85 112.25) (width 0.3) (layer F.Cu) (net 16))
 (segment (start 87.94372 112.251998) (end 80.85 112.251998) (width 0.3) (layer F.Cu) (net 16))
 (segment (start 88.945718 111.25) (end 87.94372 112.251998) (width 0.3) (layer F.Cu) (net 16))
 (segment (start 80.85 112.75) (end 88.25 112.75) (width 0.3) (layer F.Cu) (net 15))
 (segment (start 91.15 111.751998) (end 91.15 111.75) (width 0.3) (layer F.Cu) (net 15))
 (segment (start 89.248002 111.751998) (end 91.15 111.751998) (width 0.3) (layer F.Cu) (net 15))
 (segment (start 88.25 112.75) (end 89.248002 111.751998) (width 0.3) (layer F.Cu) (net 15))
 (segment (start 91.15 112.25) (end 89.95 112.25) (width 0.3) (layer F.Cu) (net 13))
 (segment (start 80.85 115.251998) (end 80.85 115.25) (width 0.3) (layer F.Cu) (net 13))
 (segment (start 79.148002 115.251998) (end 80.85 115.251998) (width 0.3) (layer F.Cu) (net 13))
 (segment (start 79.1 115.3) (end 79.148002 115.251998) (width 0.3) (layer F.Cu) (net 13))
 (via (at 79.1 115.3) (size 0.889) (layers F.Cu B.Cu) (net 13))
 (segment (start 79.1 113.7) (end 79.1 115.3) (width 0.3) (layer B.Cu) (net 13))
 (segment (start 80.1 112.7) (end 79.1 113.7) (width 0.3) (layer B.Cu) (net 13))
 (segment (start 89.5 112.7) (end 80.1 112.7) (width 0.3) (layer B.Cu) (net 13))
 (via (at 89.5 112.7) (size 0.889) (layers F.Cu B.Cu) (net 13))
 (segment (start 89.95 112.25) (end 89.5 112.7) (width 0.3) (layer F.Cu) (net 13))
 (segment (start 80.85 115.75) (end 82.75 115.75) (width 0.3) (layer F.Cu) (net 12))
 (segment (start 92.85 112.75) (end 91.15 112.75) (width 0.3) (layer F.Cu) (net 12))
 (segment (start 92.9 112.8) (end 92.85 112.75) (width 0.3) (layer F.Cu) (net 12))
 (via (at 92.9 112.8) (size 0.889) (layers F.Cu B.Cu) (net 12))
 (segment (start 92.9 114) (end 92.9 112.8) (width 0.3) (layer B.Cu) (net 12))
 (segment (start 91.6 115.3) (end 92.9 114) (width 0.3) (layer B.Cu) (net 12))
 (segment (start 83.2 115.3) (end 91.6 115.3) (width 0.3) (layer B.Cu) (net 12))
 (via (at 83.2 115.3) (size 0.889) (layers F.Cu B.Cu) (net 12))
 (segment (start 82.75 115.75) (end 83.2 115.3) (width 0.3) (layer F.Cu) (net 12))
 (segment (start 80.85 116.25) (end 83.845718 116.25) (width 0.3) (layer F.Cu) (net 11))
 (segment (start 91.15 115.251998) (end 91.15 115.25) (width 0.3) (layer F.Cu) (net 11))
 (segment (start 84.84372 115.251998) (end 91.15 115.251998) (width 0.3) (layer F.Cu) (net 11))
 (segment (start 83.845718 116.25) (end 84.84372 115.251998) (width 0.3) (layer F.Cu) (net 11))
 (segment (start 80.85 116.75) (end 84.05 116.75) (width 0.3) (layer F.Cu) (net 9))
 (segment (start 85.05 115.75) (end 91.15 115.75) (width 0.3) (layer F.Cu) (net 9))
 (segment (start 84.05 116.75) (end 85.05 115.75) (width 0.3) (layer F.Cu) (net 9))
 (segment (start 96 111.75) (end 92.95 111.75) (width 0.3) (layer F.Cu) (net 7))
 (segment (start 92.95 111.75) (end 92.7 111.5) (width 0.3) (layer F.Cu) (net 7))
 (segment (start 96.85 111.25) (end 96.85 111.751998) (width 0.3) (layer F.Cu) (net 7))
 (segment (start 96.85 111.751998) (end 96.85 111.75) (width 0.3) (layer F.Cu) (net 7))
 (segment (start 91.15 110.25) (end 91.15 110.751998) (width 0.3) (layer F.Cu) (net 7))
 (segment (start 91.15 110.751998) (end 91.15 110.75) (width 0.3) (layer F.Cu) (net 7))
 (segment (start 75.15 109.25) (end 75.15 109.75) (width 0.3) (layer F.Cu) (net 7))
 (segment (start 75.15 117.25) (end 75.15 117.75) (width 0.3) (layer F.Cu) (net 7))
 (segment (start 75.15 117.75) (end 73.45 117.75) (width 0.3) (layer F.Cu) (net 7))
 (segment (start 73.45 117.75) (end 71.9 116.2) (width 0.3) (layer F.Cu) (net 7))
 (via (at 71.9 116.2) (size 0.889) (layers F.Cu B.Cu) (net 7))
 (segment (start 71.9 116.2) (end 73.2 116.2) (width 0.3) (layer B.Cu) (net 7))
 (segment (start 73.2 116.2) (end 77.9 111.5) (width 0.3) (layer B.Cu) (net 7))
 (segment (start 77.9 111.5) (end 92.7 111.5) (width 0.3) (layer B.Cu) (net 7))
 (via (at 92.7 111.5) (size 0.889) (layers F.Cu B.Cu) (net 7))
 (segment (start 91.951998 110.751998) (end 91.15 110.751998) (width 0.3) (layer F.Cu) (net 7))
 (segment (start 92.7 111.5) (end 91.951998 110.751998) (width 0.3) (layer F.Cu) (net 7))
 (segment (start 91.15 110.751998) (end 91.15 110.75) (width 0.3) (layer F.Cu) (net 7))
 (segment (start 75.15 117.25) (end 73.85 117.25) (width 0.3) (layer F.Cu) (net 7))
 (segment (start 88.75 110.25) (end 91.15 110.25) (width 0.3) (layer F.Cu) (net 7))
 (segment (start 88.4 110.6) (end 88.75 110.25) (width 0.3) (layer F.Cu) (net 7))
 (via (at 88.4 110.6) (size 0.889) (layers F.Cu B.Cu) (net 7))
 (segment (start 77 110.6) (end 88.4 110.6) (width 0.3) (layer B.Cu) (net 7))
 (segment (start 73.2 114.4) (end 77 110.6) (width 0.3) (layer B.Cu) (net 7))
 (via (at 73.2 114.4) (size 0.889) (layers F.Cu B.Cu) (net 7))
 (segment (start 73.2 116.6) (end 73.2 114.4) (width 0.3) (layer F.Cu) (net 7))
 (segment (start 73.85 117.25) (end 73.2 116.6) (width 0.3) (layer F.Cu) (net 7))
 (segment (start 75.15 109.25) (end 78.35 109.25) (width 0.3) (layer F.Cu) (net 7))
 (segment (start 95.45 111.25) (end 96.85 111.25) (width 0.3) (layer F.Cu) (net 7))
 (segment (start 91.3 107.1) (end 95.45 111.25) (width 0.3) (layer F.Cu) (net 7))
 (segment (start 80.5 107.1) (end 91.3 107.1) (width 0.3) (layer F.Cu) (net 7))
 (segment (start 78.35 109.25) (end 80.5 107.1) (width 0.3) (layer F.Cu) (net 7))
 (segment (start 75.15 109.75) (end 78.55 109.75) (width 0.3) (layer F.Cu) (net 7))
 (segment (start 91 107.6) (end 95.15 111.75) (width 0.3) (layer F.Cu) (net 7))
 (segment (start 80.7 107.6) (end 91 107.6) (width 0.3) (layer F.Cu) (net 7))
 (segment (start 78.55 109.75) (end 80.7 107.6) (width 0.3) (layer F.Cu) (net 7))
 (segment (start 95.15 111.75) (end 96 111.75) (width 0.3) (layer F.Cu) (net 7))
 (segment (start 96 111.75) (end 96.85 111.75) (width 0.3) (layer F.Cu) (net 7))
 (segment (start 96.85 116.25) (end 96.85 116.75) (width 0.3) (layer F.Cu) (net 10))
 (segment (start 91.15 117.25) (end 91.15 117.751998) (width 0.3) (layer F.Cu) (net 10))
 (segment (start 91.15 117.751998) (end 91.15 117.75) (width 0.3) (layer F.Cu) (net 10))
 (segment (start 75.15 115.25) (end 75.15 115.75) (width 0.3) (layer F.Cu) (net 10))
 (segment (start 75.15 115.75) (end 75.15 116.25) (width 0.3) (layer F.Cu) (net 10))
 (segment (start 75.15 116.75) (end 75.15 116.25) (width 0.3) (layer F.Cu) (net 10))
 (segment (start 75.15 116.75) (end 76.15 116.75) (width 0.3) (layer F.Cu) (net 10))
 (segment (start 76.15 116.75) (end 81.1 121.7) (width 0.3) (layer F.Cu) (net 10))
 (segment (start 81.1 121.7) (end 84.7 121.7) (width 0.3) (layer F.Cu) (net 10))
 (segment (start 84.7 121.7) (end 88.648002 117.751998) (width 0.3) (layer F.Cu) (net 10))
 (segment (start 88.648002 117.751998) (end 91.15 117.751998) (width 0.3) (layer F.Cu) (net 10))
 (segment (start 91.15 117.751998) (end 91.15 117.75) (width 0.3) (layer F.Cu) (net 10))
 (segment (start 75.15 116.25) (end 76.35 116.25) (width 0.3) (layer F.Cu) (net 10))
 (segment (start 88.45 117.25) (end 91.15 117.25) (width 0.3) (layer F.Cu) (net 10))
 (segment (start 84.6 121.1) (end 88.45 117.25) (width 0.3) (layer F.Cu) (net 10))
 (segment (start 81.2 121.1) (end 84.6 121.1) (width 0.3) (layer F.Cu) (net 10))
 (segment (start 76.35 116.25) (end 81.2 121.1) (width 0.3) (layer F.Cu) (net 10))
 (segment (start 75.15 115.75) (end 76.35 115.75) (width 0.3) (layer F.Cu) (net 10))
 (segment (start 93.55 116.75) (end 96.85 116.75) (width 0.3) (layer F.Cu) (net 10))
 (segment (start 93.2 117.1) (end 93.55 116.75) (width 0.3) (layer F.Cu) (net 10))
 (via (at 93.2 117.1) (size 0.889) (layers F.Cu B.Cu) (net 10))
 (segment (start 78.3 117.1) (end 93.2 117.1) (width 0.3) (layer B.Cu) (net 10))
 (segment (start 78.2 117) (end 78.3 117.1) (width 0.3) (layer B.Cu) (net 10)) (via (at 78.2 117) (size 0.889) (layers F.Cu B.Cu) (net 10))
 (segment (start 76.35 115.75) (end 78.2 117) (width 0.3) (layer F.Cu) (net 10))
 (segment (start 75.15 115.25) (end 77.25 115.25) (width 0.3) (layer F.Cu) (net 10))
 (segment (start 94.05 116.25) (end 96.85 116.25) (width 0.3) (layer F.Cu) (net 10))
 (segment (start 93.2 115.4) (end 94.05 116.25) (width 0.3) (layer F.Cu) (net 10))
 (via (at 93.2 115.4) (size 0.889) (layers F.Cu B.Cu) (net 10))
 (segment (start 92.3 116.3) (end 93.2 115.4) (width 0.3) (layer B.Cu) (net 10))
 (segment (start 78.3 116.3) (end 92.3 116.3) (width 0.3) (layer B.Cu) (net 10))
 (segment (start 77.7 115.3) (end 78.3 116.3) (width 0.3) (layer B.Cu) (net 10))
 (via (at 77.7 115.3) (size 0.889) (layers F.Cu B.Cu) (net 10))
 (segment (start 77.25 115.25) (end 77.7 115.3) (width 0.3) (layer F.Cu) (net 10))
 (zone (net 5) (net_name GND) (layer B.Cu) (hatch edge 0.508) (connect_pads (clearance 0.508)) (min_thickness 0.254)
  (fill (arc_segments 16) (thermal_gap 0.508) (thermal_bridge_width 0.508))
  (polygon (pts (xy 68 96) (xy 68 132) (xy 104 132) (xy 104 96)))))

